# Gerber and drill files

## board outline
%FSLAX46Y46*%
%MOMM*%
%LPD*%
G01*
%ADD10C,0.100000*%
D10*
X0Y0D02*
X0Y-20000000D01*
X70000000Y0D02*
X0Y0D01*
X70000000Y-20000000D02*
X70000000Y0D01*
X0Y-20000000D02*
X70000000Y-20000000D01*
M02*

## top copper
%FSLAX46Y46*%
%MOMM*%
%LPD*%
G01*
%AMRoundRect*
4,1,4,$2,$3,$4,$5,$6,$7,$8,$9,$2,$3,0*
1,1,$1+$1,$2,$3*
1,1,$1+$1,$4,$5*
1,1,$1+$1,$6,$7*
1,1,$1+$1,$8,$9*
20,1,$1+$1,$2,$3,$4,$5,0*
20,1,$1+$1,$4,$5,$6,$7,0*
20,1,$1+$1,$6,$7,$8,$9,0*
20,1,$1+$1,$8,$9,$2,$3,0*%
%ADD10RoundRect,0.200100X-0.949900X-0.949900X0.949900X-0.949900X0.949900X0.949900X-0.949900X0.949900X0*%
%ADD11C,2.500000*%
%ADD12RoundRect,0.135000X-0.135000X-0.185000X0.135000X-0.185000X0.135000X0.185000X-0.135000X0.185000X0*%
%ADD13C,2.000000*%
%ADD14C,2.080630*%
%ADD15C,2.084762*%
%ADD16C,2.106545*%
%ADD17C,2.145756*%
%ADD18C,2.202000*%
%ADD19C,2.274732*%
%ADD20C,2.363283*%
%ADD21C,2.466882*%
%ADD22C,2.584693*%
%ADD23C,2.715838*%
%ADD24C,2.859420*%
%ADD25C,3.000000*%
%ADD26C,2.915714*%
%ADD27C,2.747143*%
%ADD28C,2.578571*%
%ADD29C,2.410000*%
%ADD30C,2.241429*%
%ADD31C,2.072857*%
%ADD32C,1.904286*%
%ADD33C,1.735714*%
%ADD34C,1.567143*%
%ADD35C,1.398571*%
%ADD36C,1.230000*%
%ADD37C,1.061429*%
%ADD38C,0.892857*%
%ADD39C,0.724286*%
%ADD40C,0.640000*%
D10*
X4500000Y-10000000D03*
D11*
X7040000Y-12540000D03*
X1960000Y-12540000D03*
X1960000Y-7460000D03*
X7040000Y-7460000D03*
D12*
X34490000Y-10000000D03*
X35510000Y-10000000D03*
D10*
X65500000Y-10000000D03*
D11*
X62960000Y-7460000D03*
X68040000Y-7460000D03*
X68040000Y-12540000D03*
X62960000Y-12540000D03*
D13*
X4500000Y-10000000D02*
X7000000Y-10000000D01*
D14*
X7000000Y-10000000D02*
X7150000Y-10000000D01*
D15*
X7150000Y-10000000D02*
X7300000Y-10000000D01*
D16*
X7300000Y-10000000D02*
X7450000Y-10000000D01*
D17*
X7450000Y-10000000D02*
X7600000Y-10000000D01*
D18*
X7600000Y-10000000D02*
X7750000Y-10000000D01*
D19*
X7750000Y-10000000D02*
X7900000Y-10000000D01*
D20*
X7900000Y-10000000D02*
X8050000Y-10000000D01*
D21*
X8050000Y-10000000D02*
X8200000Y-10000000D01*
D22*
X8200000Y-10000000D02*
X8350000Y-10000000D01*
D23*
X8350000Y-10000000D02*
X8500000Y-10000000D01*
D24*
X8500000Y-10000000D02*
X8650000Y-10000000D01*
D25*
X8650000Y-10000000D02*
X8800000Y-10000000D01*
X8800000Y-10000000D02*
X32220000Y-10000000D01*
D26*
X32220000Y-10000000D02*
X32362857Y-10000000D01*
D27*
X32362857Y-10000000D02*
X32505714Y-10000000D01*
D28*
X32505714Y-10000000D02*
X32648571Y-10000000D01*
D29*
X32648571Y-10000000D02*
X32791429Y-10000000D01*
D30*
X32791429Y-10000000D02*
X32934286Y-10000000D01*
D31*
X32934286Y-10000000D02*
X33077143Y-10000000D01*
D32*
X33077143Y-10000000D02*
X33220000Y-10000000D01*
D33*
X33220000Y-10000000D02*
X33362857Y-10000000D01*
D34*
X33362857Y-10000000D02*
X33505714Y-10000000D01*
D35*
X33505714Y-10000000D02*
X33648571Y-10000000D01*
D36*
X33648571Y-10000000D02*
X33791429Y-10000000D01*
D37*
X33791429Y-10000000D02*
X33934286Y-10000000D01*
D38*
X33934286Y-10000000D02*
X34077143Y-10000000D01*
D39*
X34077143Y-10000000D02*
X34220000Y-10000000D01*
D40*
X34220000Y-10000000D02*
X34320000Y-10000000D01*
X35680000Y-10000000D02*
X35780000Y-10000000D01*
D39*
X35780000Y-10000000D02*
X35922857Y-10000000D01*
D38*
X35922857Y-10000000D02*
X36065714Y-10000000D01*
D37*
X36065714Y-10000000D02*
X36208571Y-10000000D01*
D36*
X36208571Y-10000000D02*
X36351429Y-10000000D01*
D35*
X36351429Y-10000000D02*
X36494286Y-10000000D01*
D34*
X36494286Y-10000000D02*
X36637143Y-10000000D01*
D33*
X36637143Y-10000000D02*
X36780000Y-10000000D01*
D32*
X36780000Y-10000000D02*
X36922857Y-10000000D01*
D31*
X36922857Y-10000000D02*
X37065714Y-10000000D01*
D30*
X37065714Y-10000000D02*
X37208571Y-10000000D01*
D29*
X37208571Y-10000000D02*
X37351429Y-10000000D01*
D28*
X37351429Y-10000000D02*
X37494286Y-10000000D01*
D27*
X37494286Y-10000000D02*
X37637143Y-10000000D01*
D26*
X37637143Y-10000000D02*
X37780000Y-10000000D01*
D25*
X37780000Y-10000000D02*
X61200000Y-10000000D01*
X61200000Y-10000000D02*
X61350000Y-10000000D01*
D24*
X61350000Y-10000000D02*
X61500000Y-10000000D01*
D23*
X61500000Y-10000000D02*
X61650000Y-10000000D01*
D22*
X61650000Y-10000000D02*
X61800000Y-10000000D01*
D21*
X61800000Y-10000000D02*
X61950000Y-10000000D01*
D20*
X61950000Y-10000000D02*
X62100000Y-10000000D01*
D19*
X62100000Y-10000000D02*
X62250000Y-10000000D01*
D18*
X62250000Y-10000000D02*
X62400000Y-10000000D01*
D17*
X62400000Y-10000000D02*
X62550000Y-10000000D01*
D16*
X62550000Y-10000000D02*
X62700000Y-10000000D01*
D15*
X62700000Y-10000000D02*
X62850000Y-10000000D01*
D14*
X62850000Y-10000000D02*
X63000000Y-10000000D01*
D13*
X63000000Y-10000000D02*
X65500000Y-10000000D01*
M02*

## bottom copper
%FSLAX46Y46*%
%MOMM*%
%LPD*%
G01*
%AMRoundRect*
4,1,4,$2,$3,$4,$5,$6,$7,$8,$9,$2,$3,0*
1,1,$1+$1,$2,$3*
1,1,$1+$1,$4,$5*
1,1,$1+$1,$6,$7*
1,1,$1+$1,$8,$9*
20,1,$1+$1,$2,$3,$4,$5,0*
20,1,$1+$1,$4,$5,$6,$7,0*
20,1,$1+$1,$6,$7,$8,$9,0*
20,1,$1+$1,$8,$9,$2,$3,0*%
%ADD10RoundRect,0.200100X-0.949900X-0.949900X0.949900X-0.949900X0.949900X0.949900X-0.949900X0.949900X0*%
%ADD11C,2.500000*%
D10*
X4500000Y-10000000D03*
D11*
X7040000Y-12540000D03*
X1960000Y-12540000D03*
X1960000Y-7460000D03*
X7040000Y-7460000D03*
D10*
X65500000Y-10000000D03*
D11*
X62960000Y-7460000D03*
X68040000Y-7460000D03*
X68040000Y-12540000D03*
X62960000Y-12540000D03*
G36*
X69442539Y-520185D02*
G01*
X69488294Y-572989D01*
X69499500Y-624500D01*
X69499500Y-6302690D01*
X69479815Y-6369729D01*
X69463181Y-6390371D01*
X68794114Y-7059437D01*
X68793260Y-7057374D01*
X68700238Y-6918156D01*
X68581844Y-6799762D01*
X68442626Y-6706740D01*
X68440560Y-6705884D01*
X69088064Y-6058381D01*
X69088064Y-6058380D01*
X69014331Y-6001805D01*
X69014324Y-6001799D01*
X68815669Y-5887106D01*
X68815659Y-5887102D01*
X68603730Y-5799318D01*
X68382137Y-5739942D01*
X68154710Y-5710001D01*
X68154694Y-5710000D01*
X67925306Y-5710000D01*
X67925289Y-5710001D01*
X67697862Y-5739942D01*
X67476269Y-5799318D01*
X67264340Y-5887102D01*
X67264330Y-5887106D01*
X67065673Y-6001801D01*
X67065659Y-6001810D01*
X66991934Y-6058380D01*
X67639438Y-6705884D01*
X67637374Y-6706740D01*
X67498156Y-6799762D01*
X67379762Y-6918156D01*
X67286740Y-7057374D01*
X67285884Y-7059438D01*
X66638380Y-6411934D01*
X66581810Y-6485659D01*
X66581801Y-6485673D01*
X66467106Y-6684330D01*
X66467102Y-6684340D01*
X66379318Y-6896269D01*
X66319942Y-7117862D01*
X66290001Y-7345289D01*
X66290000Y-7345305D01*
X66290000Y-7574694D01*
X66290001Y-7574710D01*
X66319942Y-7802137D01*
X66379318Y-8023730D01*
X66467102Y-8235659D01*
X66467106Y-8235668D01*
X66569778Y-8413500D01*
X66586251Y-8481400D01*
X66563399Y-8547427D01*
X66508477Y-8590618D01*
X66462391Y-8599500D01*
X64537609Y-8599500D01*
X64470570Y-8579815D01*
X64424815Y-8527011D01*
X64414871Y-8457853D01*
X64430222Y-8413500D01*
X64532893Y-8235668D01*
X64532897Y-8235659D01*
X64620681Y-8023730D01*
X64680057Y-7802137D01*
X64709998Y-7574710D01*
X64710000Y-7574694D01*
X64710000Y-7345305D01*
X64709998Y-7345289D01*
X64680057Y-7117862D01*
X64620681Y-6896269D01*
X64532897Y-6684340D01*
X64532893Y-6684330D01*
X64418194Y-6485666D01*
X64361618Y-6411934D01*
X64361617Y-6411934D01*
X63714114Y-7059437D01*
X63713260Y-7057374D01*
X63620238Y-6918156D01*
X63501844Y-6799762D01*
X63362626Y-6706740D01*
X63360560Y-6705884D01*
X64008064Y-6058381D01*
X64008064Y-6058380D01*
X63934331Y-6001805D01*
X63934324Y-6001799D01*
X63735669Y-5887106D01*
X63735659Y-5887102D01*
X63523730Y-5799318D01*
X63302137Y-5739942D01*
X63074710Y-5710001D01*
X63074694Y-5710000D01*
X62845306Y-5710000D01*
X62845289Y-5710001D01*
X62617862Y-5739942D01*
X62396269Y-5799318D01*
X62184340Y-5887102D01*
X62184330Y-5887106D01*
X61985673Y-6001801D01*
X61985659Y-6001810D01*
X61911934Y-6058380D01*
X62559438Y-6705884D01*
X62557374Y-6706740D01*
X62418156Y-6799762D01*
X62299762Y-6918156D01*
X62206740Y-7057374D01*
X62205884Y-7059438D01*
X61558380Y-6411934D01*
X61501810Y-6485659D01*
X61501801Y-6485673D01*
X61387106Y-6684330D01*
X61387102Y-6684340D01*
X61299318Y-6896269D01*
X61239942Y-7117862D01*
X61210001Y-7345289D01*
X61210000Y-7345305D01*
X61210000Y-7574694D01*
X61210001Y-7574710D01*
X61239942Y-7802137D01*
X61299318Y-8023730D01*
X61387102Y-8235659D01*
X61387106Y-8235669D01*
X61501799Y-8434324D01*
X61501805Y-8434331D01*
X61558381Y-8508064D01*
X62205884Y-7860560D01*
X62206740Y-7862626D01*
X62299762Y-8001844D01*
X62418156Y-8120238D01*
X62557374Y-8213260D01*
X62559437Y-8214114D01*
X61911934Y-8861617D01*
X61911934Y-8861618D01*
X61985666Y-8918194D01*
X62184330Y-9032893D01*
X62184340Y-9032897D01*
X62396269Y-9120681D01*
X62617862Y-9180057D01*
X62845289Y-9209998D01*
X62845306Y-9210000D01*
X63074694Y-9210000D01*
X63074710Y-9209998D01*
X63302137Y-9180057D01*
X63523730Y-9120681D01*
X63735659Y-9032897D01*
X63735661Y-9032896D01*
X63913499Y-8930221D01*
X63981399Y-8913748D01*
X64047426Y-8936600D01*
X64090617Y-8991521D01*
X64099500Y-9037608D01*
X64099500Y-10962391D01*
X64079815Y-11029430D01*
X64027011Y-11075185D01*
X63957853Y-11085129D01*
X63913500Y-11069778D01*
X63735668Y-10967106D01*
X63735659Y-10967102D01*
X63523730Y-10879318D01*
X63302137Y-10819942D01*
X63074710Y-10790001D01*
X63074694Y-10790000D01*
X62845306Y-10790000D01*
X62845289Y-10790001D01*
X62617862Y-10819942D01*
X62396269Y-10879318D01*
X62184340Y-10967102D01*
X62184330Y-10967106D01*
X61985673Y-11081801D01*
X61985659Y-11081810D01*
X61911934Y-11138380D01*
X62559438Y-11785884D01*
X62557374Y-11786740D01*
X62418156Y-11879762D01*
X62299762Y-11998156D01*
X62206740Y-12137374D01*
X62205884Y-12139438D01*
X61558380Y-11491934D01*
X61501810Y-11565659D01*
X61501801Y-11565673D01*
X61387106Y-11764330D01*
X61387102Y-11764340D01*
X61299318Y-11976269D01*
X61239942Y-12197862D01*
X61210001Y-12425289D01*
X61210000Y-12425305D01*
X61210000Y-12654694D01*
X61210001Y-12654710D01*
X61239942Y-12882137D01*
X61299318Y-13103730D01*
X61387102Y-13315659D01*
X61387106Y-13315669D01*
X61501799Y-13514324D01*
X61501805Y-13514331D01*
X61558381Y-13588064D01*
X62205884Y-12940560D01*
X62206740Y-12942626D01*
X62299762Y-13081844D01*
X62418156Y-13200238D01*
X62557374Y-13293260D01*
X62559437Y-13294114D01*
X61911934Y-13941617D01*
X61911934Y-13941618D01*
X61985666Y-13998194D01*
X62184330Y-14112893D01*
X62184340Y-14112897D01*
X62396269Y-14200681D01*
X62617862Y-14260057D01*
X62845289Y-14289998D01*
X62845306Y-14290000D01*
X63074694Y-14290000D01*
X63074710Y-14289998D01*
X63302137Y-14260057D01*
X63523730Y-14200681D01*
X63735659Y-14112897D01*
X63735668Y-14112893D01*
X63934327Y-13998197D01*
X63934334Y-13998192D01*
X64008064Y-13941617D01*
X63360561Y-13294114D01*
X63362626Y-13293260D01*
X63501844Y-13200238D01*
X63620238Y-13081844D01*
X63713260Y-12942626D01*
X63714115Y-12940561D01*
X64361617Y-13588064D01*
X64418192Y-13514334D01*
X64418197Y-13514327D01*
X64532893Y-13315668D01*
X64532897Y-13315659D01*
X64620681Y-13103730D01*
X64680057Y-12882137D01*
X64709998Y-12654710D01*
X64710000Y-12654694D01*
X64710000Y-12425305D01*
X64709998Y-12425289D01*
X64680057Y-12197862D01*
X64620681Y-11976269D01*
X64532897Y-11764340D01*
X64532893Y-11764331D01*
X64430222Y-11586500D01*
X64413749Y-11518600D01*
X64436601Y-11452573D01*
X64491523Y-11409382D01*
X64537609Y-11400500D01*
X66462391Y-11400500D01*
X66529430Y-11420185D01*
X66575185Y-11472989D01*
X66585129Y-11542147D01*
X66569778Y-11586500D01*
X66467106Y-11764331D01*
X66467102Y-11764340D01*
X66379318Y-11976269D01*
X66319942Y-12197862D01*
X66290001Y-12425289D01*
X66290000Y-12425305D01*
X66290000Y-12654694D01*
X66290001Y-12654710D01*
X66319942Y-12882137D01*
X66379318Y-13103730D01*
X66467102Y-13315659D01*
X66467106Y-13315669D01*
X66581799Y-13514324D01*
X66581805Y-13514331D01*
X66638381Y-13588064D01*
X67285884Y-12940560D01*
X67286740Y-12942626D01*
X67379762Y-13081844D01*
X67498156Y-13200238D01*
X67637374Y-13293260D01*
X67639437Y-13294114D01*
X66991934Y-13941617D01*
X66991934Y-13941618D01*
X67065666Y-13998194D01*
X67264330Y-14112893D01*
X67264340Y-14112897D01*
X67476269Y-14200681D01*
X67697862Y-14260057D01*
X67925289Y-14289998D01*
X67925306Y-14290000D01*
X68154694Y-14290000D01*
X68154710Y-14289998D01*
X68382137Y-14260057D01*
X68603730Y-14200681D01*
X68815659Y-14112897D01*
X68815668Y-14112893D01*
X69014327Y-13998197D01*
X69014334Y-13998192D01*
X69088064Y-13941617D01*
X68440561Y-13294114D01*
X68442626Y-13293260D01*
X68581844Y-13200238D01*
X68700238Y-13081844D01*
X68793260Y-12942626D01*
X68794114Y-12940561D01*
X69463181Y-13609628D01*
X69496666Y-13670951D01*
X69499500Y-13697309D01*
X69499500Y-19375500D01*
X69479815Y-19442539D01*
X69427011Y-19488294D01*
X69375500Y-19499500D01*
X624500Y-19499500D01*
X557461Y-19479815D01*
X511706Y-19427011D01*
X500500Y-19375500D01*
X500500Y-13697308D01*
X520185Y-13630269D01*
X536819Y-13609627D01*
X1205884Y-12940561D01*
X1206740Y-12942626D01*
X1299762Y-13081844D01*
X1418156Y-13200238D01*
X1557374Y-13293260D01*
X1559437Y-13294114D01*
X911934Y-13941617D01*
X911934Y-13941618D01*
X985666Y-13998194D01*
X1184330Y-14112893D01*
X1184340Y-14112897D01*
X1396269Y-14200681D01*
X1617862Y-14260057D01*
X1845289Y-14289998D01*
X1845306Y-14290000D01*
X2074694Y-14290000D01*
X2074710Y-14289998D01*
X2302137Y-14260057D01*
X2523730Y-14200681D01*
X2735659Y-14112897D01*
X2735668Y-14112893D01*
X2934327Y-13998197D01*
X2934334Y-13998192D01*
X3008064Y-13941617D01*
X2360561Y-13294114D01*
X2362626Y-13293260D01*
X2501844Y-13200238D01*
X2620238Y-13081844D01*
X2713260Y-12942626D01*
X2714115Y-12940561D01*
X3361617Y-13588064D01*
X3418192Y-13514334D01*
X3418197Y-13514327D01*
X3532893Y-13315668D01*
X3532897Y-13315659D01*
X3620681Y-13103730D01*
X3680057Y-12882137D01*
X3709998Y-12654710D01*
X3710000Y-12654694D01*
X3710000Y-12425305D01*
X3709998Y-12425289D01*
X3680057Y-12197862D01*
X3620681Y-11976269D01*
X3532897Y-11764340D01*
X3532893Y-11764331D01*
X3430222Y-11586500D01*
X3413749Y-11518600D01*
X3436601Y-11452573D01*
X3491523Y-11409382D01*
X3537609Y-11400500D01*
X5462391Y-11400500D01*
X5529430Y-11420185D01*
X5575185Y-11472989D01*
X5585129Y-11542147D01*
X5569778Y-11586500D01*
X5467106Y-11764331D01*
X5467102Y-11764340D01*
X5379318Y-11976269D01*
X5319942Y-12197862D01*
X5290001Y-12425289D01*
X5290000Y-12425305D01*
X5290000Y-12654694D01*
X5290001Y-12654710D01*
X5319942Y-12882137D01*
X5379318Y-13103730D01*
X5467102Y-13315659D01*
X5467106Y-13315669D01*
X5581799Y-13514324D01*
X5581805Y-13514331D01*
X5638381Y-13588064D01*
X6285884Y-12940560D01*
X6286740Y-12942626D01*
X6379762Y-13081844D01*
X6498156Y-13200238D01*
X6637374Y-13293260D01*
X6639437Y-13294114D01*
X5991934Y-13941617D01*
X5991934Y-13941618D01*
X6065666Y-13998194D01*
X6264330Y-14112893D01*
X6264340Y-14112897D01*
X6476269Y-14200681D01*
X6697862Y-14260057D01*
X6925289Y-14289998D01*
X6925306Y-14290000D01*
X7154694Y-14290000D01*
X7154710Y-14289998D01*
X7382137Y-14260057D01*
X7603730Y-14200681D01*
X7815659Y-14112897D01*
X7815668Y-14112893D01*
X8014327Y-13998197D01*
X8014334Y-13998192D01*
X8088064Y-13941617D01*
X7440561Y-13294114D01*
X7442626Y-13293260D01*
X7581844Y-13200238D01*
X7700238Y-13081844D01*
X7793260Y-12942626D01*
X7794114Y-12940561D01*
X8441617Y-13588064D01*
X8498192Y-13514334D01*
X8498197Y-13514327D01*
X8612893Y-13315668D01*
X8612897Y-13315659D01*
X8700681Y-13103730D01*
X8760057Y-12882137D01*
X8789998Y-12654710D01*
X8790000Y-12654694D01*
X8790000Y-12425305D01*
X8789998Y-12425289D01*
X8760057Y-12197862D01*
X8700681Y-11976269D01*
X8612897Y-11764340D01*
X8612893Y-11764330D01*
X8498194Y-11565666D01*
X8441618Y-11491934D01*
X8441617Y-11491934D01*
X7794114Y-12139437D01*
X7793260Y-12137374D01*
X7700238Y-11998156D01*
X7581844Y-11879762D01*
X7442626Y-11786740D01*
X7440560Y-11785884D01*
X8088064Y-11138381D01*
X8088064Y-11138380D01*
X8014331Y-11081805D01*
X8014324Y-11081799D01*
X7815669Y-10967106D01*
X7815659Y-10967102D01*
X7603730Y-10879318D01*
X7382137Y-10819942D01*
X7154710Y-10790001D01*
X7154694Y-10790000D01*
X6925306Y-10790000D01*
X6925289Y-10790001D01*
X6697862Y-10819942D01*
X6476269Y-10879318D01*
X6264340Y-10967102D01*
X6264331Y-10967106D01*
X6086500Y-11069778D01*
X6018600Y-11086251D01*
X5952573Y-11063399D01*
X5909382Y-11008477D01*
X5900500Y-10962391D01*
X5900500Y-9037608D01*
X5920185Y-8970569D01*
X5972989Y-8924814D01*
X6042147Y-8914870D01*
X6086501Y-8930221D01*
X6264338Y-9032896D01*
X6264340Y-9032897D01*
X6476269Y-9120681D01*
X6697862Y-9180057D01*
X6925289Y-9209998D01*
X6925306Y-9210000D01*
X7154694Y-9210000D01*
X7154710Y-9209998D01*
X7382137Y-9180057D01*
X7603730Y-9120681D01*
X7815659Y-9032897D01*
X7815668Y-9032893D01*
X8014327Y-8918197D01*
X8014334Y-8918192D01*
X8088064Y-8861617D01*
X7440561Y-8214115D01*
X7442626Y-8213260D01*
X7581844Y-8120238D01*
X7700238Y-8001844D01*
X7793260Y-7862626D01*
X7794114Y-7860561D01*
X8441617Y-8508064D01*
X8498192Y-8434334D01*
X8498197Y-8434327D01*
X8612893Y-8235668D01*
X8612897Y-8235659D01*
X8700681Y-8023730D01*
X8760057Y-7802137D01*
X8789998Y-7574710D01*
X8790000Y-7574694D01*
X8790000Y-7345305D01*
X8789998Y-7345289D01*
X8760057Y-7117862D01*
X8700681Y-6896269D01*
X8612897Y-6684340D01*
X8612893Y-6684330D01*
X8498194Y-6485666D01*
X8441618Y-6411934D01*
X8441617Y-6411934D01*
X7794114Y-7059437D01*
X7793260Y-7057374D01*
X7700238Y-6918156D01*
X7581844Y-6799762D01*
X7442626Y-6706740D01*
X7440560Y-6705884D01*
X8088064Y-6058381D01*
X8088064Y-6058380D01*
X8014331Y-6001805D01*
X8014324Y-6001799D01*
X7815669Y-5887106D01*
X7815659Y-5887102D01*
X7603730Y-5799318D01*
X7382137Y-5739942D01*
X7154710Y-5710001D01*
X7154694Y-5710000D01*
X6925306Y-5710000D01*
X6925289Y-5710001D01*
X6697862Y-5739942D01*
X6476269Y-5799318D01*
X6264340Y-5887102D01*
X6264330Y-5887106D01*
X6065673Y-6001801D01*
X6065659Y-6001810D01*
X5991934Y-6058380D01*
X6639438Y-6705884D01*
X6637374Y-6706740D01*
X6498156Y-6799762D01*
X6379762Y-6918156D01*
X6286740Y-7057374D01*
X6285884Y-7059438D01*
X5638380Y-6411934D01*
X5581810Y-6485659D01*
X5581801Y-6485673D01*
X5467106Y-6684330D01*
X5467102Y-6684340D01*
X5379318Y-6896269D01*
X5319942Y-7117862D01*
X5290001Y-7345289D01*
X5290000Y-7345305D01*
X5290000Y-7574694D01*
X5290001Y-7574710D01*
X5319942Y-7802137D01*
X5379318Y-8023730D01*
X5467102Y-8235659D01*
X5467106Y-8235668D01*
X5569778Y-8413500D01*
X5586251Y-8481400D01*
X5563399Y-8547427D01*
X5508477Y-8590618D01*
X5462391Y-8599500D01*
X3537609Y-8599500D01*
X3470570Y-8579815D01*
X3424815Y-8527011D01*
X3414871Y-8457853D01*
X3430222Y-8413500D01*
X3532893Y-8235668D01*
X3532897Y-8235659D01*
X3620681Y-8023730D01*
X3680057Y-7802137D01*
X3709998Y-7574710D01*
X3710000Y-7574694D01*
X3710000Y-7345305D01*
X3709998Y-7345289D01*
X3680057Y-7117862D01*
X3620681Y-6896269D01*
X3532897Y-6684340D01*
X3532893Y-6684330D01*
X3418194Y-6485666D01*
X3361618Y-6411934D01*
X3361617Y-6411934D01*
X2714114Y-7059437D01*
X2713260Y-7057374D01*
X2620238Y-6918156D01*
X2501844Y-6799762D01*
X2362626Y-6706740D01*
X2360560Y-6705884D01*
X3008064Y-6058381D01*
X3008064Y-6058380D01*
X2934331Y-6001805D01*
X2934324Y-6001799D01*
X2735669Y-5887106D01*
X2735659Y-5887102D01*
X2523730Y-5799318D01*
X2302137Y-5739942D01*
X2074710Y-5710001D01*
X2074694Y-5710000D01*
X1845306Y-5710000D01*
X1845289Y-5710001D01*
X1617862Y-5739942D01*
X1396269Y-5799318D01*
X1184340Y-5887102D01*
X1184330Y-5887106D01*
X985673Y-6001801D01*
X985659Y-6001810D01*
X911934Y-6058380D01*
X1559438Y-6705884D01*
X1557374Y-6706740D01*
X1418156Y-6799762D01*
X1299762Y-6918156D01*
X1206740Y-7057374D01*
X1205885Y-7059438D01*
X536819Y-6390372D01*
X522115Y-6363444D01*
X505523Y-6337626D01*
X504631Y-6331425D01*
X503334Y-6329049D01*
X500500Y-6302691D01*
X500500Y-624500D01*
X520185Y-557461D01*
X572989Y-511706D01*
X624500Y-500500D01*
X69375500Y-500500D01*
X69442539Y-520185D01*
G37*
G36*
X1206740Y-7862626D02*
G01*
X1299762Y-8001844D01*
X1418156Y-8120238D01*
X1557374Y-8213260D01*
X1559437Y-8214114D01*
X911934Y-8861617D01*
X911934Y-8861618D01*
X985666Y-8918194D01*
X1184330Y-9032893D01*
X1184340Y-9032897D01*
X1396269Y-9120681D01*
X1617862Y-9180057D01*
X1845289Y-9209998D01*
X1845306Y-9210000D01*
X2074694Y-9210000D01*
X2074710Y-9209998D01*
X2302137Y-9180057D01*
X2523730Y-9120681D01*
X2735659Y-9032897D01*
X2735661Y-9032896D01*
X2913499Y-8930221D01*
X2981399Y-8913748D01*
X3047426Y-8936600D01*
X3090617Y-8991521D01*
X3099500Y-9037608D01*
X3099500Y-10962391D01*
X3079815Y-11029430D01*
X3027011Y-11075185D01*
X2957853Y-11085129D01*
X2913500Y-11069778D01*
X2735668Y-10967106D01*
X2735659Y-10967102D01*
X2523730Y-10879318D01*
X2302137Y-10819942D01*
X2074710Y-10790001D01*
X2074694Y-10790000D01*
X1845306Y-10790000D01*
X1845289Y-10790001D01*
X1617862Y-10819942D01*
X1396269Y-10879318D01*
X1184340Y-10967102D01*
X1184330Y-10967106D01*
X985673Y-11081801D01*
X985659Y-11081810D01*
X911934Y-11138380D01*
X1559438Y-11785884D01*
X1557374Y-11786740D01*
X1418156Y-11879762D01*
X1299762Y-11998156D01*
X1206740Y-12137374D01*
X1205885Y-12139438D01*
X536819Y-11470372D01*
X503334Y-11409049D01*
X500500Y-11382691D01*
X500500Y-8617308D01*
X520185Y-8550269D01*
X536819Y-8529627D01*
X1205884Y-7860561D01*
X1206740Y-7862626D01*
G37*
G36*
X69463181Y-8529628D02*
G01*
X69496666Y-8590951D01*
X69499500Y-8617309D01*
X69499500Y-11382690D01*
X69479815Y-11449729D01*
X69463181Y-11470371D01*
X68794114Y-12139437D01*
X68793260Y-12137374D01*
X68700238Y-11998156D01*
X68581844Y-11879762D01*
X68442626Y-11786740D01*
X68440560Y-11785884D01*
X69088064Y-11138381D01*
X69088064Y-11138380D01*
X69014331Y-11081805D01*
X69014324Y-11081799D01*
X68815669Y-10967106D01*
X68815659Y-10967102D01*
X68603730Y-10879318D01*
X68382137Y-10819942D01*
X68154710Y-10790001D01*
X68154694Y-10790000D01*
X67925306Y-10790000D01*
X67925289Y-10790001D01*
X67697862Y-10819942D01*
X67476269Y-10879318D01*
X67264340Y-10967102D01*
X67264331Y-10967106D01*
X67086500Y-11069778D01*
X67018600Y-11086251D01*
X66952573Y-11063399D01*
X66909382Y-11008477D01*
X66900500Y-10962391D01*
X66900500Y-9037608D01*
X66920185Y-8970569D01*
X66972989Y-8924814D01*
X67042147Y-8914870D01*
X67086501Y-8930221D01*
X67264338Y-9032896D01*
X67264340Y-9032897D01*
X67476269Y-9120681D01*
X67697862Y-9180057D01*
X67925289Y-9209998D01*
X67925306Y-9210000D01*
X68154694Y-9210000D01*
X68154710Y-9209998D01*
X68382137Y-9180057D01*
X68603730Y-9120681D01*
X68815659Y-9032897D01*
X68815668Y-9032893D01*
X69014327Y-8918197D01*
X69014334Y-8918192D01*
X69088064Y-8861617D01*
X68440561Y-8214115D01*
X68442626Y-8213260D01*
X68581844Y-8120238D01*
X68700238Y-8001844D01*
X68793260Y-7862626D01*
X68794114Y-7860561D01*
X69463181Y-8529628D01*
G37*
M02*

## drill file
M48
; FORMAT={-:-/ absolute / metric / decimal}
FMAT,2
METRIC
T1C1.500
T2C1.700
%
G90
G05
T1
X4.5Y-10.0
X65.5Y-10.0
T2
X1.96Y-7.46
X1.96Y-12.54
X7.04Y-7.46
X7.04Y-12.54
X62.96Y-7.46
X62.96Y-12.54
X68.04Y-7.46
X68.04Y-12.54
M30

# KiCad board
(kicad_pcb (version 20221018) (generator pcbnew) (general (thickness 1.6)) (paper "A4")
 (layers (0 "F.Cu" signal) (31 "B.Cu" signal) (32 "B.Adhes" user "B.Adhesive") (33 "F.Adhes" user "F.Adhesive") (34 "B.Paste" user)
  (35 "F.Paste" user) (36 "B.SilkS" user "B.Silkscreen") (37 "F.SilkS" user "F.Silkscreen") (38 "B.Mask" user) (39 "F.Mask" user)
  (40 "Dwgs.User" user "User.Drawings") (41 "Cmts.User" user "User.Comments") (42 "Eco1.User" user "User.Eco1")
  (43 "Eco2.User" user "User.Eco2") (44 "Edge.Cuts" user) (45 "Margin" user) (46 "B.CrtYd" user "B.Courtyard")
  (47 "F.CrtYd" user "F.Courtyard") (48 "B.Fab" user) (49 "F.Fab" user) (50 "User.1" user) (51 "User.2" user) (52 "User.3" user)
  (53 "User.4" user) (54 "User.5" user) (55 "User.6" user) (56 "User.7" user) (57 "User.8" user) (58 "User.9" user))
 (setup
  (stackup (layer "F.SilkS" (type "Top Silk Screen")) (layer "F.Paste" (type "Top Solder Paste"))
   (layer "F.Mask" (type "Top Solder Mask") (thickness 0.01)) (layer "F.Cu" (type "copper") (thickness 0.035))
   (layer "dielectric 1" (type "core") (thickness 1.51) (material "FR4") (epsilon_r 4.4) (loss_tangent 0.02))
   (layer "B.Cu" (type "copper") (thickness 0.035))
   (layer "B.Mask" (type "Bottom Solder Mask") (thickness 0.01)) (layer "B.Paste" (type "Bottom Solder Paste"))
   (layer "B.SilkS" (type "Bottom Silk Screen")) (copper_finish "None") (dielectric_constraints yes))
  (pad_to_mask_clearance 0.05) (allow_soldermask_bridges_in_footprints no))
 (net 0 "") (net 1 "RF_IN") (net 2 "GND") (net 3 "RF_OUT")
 (gr_line (start 0 0) (end 0 20) (layer "Edge.Cuts") (width 0.1))
 (gr_line (start 70 0) (end 0 0) (layer "Edge.Cuts") (width 0.1))
 (gr_line (start 70 20) (end 70 0) (layer "Edge.Cuts") (width 0.1))
 (gr_line (start 0 20) (end 70 20) (layer "Edge.Cuts") (width 0.1))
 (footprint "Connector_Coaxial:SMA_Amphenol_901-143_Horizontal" (layer "F.Cu") (at 4.5 10 90)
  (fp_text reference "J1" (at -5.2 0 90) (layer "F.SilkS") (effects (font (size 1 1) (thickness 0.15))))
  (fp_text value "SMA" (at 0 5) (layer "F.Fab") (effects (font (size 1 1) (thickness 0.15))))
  (pad "1" thru_hole roundrect (at 0 0) (size 2.3 2.3) (drill 1.5) (layers *.Cu *.Mask) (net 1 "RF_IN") (remove_unused_layers)
   (keep_end_layers) (roundrect_rratio 0.087))
  (pad "2" thru_hole circle (at -2.54 2.54) (size 2.5 2.5) (drill 1.7) (layers *.Cu *.Mask) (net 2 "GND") (remove_unused_layers)
   (keep_end_layers))
  (pad "2" thru_hole circle (at -2.54 -2.54) (size 2.5 2.5) (drill 1.7) (layers *.Cu *.Mask) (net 2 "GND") (remove_unused_layers)
   (keep_end_layers))
  (pad "2" thru_hole circle (at 2.54 -2.54) (size 2.5 2.5) (drill 1.7) (layers *.Cu *.Mask) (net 2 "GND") (remove_unused_layers)
   (keep_end_layers))
  (pad "2" thru_hole circle (at 2.54 2.54) (size 2.5 2.5) (drill 1.7) (layers *.Cu *.Mask) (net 2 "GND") (remove_unused_layers)
   (keep_end_layers)))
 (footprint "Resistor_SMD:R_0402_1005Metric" (layer "F.Cu") (at 35 10)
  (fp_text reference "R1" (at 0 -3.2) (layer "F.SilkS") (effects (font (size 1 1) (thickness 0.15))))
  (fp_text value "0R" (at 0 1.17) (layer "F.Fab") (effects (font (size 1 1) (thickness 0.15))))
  (pad "1" smd roundrect (at -0.51 0) (size 0.54 0.64) (layers "F.Cu" "F.Paste" "F.Mask") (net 1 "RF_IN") (roundrect_rratio 0.25))
  (pad "2" smd roundrect (at 0.51 0) (size 0.54 0.64) (layers "F.Cu" "F.Paste" "F.Mask") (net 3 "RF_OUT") (roundrect_rratio 0.25)))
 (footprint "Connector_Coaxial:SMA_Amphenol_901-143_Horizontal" (layer "F.Cu") (at 65.5 10 270)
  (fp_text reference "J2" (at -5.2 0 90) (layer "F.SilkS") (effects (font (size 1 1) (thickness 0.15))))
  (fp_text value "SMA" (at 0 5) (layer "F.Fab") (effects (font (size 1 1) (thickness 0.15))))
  (pad "1" thru_hole roundrect (at 0 0) (size 2.3 2.3) (drill 1.5) (layers *.Cu *.Mask) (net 3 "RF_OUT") (remove_unused_layers)
   (keep_end_layers) (roundrect_rratio 0.087))
  (pad "2" thru_hole circle (at -2.54 2.54) (size 2.5 2.5) (drill 1.7) (layers *.Cu *.Mask) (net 2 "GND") (remove_unused_layers)
   (keep_end_layers))
  (pad "2" thru_hole circle (at -2.54 -2.54) (size 2.5 2.5) (drill 1.7) (layers *.Cu *.Mask) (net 2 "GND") (remove_unused_layers)
   (keep_end_layers))
  (pad "2" thru_hole circle (at 2.54 -2.54) (size 2.5 2.5) (drill 1.7) (layers *.Cu *.Mask) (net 2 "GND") (remove_unused_layers)
   (keep_end_layers))
  (pad "2" thru_hole circle (at 2.54 2.54) (size 2.5 2.5) (drill 1.7) (layers *.Cu *.Mask) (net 2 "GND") (remove_unused_layers)
   (keep_end_layers)))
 (segment (start 4.5 10) (end 7 10) (width 2) (layer "F.Cu") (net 1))
 (segment (start 7 10) (end 7.15 10) (width 2.08063) (layer "F.Cu") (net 1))
 (segment (start 7.15 10) (end 7.3 10) (width 2.084762) (layer "F.Cu") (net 1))
 (segment (start 7.3 10) (end 7.45 10) (width 2.106545) (layer "F.Cu") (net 1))
 (segment (start 7.45 10) (end 7.6 10) (width 2.145756) (layer "F.Cu") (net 1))
 (segment (start 7.6 10) (end 7.75 10) (width 2.202) (layer "F.Cu") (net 1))
 (segment (start 7.75 10) (end 7.9 10) (width 2.274732) (layer "F.Cu") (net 1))
 (segment (start 7.9 10) (end 8.05 10) (width 2.363283) (layer "F.Cu") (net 1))
 (segment (start 8.05 10) (end 8.2 10) (width 2.466882) (layer "F.Cu") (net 1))
 (segment (start 8.2 10) (end 8.35 10) (width 2.584693) (layer "F.Cu") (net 1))
 (segment (start 8.35 10) (end 8.5 10) (width 2.715838) (layer "F.Cu") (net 1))
 (segment (start 8.5 10) (end 8.65 10) (width 2.85942) (layer "F.Cu") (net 1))
 (segment (start 8.65 10) (end 8.8 10) (width 3) (layer "F.Cu") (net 1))
 (segment (start 8.8 10) (end 32.22 10) (width 3) (layer "F.Cu") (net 1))
 (segment (start 32.22 10) (end 32.362857 10) (width 2.915714) (layer "F.Cu") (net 1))
 (segment (start 32.362857 10) (end 32.505714 10) (width 2.747143) (layer "F.Cu") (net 1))
 (segment (start 32.505714 10) (end 32.648571 10) (width 2.578571) (layer "F.Cu") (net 1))
 (segment (start 32.648571 10) (end 32.791429 10) (width 2.41) (layer "F.Cu") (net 1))
 (segment (start 32.791429 10) (end 32.934286 10) (width 2.241429) (layer "F.Cu") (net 1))
 (segment (start 32.934286 10) (end 33.077143 10) (width 2.072857) (layer "F.Cu") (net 1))
 (segment (start 33.077143 10) (end 33.22 10) (width 1.904286) (layer "F.Cu") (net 1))
 (segment (start 33.22 10) (end 33.362857 10) (width 1.735714) (layer "F.Cu") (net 1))
 (segment (start 33.362857 10) (end 33.505714 10) (width 1.567143) (layer "F.Cu") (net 1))
 (segment (start 33.505714 10) (end 33.648571 10) (width 1.398571) (layer "F.Cu") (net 1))
 (segment (start 33.648571 10) (end 33.791429 10) (width 1.23) (layer "F.Cu") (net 1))
 (segment (start 33.791429 10) (end 33.934286 10) (width 1.061429) (layer "F.Cu") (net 1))
 (segment (start 33.934286 10) (end 34.077143 10) (width 0.892857) (layer "F.Cu") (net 1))
 (segment (start 34.077143 10) (end 34.22 10) (width 0.724286) (layer "F.Cu") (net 1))
 (segment (start 34.22 10) (end 34.32 10) (width 0.64) (layer "F.Cu") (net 1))
 (segment (start 35.68 10) (end 35.78 10) (width 0.64) (layer "F.Cu") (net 3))
 (segment (start 35.78 10) (end 35.922857 10) (width 0.724286) (layer "F.Cu") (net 3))
 (segment (start 35.922857 10) (end 36.065714 10) (width 0.892857) (layer "F.Cu") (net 3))
 (segment (start 36.065714 10) (end 36.208571 10) (width 1.061429) (layer "F.Cu") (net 3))
 (segment (start 36.208571 10) (end 36.351429 10) (width 1.23) (layer "F.Cu") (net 3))
 (segment (start 36.351429 10) (end 36.494286 10) (width 1.398571) (layer "F.Cu") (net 3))
 (segment (start 36.494286 10) (end 36.637143 10) (width 1.567143) (layer "F.Cu") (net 3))
 (segment (start 36.637143 10) (end 36.78 10) (width 1.735714) (layer "F.Cu") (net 3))
 (segment (start 36.78 10) (end 36.922857 10) (width 1.904286) (layer "F.Cu") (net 3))
 (segment (start 36.922857 10) (end 37.065714 10) (width 2.072857) (layer "F.Cu") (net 3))
 (segment (start 37.065714 10) (end 37.208571 10) (width 2.241429) (layer "F.Cu") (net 3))
 (segment (start 37.208571 10) (end 37.351429 10) (width 2.41) (layer "F.Cu") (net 3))
 (segment (start 37.351429 10) (end 37.494286 10) (width 2.578571) (layer "F.Cu") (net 3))
 (segment (start 37.494286 10) (end 37.637143 10) (width 2.747143) (layer "F.Cu") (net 3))
 (segment (start 37.637143 10) (end 37.78 10) (width 2.915714) (layer "F.Cu") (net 3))
 (segment (start 37.78 10) (end 61.2 10) (width 3) (layer "F.Cu") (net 3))
 (segment (start 61.2 10) (end 61.35 10) (width 3) (layer "F.Cu") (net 3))
 (segment (start 61.35 10) (end 61.5 10) (width 2.85942) (layer "F.Cu") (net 3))
 (segment (start 61.5 10) (end 61.65 10) (width 2.715838) (layer "F.Cu") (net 3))
 (segment (start 61.65 10) (end 61.8 10) (width 2.584693) (layer "F.Cu") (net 3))
 (segment (start 61.8 10) (end 61.95 10) (width 2.466882) (layer "F.Cu") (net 3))
 (segment (start 61.95 10) (end 62.1 10) (width 2.363283) (layer "F.Cu") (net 3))
 (segment (start 62.1 10) (end 62.25 10) (width 2.274732) (layer "F.Cu") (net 3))
 (segment (start 62.25 10) (end 62.4 10) (width 2.202) (layer "F.Cu") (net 3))
 (segment (start 62.4 10) (end 62.55 10) (width 2.145756) (layer "F.Cu") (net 3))
 (segment (start 62.55 10) (end 62.7 10) (width 2.106545) (layer "F.Cu") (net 3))
 (segment (start 62.7 10) (end 62.85 10) (width 2.084762) (layer "F.Cu") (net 3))
 (segment (start 62.85 10) (end 63 10) (width 2.08063) (layer "F.Cu") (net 3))
 (segment (start 63 10) (end 65.5 10) (width 2) (layer "F.Cu") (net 3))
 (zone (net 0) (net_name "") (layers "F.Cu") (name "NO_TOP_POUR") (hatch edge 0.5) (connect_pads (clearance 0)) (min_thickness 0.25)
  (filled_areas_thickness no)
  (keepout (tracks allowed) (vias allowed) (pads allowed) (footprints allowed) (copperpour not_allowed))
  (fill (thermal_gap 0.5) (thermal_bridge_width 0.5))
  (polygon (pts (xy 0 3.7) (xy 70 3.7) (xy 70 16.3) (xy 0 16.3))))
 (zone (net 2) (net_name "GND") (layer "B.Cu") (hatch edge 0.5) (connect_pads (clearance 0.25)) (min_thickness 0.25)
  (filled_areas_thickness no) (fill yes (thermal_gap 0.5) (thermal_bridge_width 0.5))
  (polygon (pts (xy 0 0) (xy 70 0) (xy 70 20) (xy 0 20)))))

